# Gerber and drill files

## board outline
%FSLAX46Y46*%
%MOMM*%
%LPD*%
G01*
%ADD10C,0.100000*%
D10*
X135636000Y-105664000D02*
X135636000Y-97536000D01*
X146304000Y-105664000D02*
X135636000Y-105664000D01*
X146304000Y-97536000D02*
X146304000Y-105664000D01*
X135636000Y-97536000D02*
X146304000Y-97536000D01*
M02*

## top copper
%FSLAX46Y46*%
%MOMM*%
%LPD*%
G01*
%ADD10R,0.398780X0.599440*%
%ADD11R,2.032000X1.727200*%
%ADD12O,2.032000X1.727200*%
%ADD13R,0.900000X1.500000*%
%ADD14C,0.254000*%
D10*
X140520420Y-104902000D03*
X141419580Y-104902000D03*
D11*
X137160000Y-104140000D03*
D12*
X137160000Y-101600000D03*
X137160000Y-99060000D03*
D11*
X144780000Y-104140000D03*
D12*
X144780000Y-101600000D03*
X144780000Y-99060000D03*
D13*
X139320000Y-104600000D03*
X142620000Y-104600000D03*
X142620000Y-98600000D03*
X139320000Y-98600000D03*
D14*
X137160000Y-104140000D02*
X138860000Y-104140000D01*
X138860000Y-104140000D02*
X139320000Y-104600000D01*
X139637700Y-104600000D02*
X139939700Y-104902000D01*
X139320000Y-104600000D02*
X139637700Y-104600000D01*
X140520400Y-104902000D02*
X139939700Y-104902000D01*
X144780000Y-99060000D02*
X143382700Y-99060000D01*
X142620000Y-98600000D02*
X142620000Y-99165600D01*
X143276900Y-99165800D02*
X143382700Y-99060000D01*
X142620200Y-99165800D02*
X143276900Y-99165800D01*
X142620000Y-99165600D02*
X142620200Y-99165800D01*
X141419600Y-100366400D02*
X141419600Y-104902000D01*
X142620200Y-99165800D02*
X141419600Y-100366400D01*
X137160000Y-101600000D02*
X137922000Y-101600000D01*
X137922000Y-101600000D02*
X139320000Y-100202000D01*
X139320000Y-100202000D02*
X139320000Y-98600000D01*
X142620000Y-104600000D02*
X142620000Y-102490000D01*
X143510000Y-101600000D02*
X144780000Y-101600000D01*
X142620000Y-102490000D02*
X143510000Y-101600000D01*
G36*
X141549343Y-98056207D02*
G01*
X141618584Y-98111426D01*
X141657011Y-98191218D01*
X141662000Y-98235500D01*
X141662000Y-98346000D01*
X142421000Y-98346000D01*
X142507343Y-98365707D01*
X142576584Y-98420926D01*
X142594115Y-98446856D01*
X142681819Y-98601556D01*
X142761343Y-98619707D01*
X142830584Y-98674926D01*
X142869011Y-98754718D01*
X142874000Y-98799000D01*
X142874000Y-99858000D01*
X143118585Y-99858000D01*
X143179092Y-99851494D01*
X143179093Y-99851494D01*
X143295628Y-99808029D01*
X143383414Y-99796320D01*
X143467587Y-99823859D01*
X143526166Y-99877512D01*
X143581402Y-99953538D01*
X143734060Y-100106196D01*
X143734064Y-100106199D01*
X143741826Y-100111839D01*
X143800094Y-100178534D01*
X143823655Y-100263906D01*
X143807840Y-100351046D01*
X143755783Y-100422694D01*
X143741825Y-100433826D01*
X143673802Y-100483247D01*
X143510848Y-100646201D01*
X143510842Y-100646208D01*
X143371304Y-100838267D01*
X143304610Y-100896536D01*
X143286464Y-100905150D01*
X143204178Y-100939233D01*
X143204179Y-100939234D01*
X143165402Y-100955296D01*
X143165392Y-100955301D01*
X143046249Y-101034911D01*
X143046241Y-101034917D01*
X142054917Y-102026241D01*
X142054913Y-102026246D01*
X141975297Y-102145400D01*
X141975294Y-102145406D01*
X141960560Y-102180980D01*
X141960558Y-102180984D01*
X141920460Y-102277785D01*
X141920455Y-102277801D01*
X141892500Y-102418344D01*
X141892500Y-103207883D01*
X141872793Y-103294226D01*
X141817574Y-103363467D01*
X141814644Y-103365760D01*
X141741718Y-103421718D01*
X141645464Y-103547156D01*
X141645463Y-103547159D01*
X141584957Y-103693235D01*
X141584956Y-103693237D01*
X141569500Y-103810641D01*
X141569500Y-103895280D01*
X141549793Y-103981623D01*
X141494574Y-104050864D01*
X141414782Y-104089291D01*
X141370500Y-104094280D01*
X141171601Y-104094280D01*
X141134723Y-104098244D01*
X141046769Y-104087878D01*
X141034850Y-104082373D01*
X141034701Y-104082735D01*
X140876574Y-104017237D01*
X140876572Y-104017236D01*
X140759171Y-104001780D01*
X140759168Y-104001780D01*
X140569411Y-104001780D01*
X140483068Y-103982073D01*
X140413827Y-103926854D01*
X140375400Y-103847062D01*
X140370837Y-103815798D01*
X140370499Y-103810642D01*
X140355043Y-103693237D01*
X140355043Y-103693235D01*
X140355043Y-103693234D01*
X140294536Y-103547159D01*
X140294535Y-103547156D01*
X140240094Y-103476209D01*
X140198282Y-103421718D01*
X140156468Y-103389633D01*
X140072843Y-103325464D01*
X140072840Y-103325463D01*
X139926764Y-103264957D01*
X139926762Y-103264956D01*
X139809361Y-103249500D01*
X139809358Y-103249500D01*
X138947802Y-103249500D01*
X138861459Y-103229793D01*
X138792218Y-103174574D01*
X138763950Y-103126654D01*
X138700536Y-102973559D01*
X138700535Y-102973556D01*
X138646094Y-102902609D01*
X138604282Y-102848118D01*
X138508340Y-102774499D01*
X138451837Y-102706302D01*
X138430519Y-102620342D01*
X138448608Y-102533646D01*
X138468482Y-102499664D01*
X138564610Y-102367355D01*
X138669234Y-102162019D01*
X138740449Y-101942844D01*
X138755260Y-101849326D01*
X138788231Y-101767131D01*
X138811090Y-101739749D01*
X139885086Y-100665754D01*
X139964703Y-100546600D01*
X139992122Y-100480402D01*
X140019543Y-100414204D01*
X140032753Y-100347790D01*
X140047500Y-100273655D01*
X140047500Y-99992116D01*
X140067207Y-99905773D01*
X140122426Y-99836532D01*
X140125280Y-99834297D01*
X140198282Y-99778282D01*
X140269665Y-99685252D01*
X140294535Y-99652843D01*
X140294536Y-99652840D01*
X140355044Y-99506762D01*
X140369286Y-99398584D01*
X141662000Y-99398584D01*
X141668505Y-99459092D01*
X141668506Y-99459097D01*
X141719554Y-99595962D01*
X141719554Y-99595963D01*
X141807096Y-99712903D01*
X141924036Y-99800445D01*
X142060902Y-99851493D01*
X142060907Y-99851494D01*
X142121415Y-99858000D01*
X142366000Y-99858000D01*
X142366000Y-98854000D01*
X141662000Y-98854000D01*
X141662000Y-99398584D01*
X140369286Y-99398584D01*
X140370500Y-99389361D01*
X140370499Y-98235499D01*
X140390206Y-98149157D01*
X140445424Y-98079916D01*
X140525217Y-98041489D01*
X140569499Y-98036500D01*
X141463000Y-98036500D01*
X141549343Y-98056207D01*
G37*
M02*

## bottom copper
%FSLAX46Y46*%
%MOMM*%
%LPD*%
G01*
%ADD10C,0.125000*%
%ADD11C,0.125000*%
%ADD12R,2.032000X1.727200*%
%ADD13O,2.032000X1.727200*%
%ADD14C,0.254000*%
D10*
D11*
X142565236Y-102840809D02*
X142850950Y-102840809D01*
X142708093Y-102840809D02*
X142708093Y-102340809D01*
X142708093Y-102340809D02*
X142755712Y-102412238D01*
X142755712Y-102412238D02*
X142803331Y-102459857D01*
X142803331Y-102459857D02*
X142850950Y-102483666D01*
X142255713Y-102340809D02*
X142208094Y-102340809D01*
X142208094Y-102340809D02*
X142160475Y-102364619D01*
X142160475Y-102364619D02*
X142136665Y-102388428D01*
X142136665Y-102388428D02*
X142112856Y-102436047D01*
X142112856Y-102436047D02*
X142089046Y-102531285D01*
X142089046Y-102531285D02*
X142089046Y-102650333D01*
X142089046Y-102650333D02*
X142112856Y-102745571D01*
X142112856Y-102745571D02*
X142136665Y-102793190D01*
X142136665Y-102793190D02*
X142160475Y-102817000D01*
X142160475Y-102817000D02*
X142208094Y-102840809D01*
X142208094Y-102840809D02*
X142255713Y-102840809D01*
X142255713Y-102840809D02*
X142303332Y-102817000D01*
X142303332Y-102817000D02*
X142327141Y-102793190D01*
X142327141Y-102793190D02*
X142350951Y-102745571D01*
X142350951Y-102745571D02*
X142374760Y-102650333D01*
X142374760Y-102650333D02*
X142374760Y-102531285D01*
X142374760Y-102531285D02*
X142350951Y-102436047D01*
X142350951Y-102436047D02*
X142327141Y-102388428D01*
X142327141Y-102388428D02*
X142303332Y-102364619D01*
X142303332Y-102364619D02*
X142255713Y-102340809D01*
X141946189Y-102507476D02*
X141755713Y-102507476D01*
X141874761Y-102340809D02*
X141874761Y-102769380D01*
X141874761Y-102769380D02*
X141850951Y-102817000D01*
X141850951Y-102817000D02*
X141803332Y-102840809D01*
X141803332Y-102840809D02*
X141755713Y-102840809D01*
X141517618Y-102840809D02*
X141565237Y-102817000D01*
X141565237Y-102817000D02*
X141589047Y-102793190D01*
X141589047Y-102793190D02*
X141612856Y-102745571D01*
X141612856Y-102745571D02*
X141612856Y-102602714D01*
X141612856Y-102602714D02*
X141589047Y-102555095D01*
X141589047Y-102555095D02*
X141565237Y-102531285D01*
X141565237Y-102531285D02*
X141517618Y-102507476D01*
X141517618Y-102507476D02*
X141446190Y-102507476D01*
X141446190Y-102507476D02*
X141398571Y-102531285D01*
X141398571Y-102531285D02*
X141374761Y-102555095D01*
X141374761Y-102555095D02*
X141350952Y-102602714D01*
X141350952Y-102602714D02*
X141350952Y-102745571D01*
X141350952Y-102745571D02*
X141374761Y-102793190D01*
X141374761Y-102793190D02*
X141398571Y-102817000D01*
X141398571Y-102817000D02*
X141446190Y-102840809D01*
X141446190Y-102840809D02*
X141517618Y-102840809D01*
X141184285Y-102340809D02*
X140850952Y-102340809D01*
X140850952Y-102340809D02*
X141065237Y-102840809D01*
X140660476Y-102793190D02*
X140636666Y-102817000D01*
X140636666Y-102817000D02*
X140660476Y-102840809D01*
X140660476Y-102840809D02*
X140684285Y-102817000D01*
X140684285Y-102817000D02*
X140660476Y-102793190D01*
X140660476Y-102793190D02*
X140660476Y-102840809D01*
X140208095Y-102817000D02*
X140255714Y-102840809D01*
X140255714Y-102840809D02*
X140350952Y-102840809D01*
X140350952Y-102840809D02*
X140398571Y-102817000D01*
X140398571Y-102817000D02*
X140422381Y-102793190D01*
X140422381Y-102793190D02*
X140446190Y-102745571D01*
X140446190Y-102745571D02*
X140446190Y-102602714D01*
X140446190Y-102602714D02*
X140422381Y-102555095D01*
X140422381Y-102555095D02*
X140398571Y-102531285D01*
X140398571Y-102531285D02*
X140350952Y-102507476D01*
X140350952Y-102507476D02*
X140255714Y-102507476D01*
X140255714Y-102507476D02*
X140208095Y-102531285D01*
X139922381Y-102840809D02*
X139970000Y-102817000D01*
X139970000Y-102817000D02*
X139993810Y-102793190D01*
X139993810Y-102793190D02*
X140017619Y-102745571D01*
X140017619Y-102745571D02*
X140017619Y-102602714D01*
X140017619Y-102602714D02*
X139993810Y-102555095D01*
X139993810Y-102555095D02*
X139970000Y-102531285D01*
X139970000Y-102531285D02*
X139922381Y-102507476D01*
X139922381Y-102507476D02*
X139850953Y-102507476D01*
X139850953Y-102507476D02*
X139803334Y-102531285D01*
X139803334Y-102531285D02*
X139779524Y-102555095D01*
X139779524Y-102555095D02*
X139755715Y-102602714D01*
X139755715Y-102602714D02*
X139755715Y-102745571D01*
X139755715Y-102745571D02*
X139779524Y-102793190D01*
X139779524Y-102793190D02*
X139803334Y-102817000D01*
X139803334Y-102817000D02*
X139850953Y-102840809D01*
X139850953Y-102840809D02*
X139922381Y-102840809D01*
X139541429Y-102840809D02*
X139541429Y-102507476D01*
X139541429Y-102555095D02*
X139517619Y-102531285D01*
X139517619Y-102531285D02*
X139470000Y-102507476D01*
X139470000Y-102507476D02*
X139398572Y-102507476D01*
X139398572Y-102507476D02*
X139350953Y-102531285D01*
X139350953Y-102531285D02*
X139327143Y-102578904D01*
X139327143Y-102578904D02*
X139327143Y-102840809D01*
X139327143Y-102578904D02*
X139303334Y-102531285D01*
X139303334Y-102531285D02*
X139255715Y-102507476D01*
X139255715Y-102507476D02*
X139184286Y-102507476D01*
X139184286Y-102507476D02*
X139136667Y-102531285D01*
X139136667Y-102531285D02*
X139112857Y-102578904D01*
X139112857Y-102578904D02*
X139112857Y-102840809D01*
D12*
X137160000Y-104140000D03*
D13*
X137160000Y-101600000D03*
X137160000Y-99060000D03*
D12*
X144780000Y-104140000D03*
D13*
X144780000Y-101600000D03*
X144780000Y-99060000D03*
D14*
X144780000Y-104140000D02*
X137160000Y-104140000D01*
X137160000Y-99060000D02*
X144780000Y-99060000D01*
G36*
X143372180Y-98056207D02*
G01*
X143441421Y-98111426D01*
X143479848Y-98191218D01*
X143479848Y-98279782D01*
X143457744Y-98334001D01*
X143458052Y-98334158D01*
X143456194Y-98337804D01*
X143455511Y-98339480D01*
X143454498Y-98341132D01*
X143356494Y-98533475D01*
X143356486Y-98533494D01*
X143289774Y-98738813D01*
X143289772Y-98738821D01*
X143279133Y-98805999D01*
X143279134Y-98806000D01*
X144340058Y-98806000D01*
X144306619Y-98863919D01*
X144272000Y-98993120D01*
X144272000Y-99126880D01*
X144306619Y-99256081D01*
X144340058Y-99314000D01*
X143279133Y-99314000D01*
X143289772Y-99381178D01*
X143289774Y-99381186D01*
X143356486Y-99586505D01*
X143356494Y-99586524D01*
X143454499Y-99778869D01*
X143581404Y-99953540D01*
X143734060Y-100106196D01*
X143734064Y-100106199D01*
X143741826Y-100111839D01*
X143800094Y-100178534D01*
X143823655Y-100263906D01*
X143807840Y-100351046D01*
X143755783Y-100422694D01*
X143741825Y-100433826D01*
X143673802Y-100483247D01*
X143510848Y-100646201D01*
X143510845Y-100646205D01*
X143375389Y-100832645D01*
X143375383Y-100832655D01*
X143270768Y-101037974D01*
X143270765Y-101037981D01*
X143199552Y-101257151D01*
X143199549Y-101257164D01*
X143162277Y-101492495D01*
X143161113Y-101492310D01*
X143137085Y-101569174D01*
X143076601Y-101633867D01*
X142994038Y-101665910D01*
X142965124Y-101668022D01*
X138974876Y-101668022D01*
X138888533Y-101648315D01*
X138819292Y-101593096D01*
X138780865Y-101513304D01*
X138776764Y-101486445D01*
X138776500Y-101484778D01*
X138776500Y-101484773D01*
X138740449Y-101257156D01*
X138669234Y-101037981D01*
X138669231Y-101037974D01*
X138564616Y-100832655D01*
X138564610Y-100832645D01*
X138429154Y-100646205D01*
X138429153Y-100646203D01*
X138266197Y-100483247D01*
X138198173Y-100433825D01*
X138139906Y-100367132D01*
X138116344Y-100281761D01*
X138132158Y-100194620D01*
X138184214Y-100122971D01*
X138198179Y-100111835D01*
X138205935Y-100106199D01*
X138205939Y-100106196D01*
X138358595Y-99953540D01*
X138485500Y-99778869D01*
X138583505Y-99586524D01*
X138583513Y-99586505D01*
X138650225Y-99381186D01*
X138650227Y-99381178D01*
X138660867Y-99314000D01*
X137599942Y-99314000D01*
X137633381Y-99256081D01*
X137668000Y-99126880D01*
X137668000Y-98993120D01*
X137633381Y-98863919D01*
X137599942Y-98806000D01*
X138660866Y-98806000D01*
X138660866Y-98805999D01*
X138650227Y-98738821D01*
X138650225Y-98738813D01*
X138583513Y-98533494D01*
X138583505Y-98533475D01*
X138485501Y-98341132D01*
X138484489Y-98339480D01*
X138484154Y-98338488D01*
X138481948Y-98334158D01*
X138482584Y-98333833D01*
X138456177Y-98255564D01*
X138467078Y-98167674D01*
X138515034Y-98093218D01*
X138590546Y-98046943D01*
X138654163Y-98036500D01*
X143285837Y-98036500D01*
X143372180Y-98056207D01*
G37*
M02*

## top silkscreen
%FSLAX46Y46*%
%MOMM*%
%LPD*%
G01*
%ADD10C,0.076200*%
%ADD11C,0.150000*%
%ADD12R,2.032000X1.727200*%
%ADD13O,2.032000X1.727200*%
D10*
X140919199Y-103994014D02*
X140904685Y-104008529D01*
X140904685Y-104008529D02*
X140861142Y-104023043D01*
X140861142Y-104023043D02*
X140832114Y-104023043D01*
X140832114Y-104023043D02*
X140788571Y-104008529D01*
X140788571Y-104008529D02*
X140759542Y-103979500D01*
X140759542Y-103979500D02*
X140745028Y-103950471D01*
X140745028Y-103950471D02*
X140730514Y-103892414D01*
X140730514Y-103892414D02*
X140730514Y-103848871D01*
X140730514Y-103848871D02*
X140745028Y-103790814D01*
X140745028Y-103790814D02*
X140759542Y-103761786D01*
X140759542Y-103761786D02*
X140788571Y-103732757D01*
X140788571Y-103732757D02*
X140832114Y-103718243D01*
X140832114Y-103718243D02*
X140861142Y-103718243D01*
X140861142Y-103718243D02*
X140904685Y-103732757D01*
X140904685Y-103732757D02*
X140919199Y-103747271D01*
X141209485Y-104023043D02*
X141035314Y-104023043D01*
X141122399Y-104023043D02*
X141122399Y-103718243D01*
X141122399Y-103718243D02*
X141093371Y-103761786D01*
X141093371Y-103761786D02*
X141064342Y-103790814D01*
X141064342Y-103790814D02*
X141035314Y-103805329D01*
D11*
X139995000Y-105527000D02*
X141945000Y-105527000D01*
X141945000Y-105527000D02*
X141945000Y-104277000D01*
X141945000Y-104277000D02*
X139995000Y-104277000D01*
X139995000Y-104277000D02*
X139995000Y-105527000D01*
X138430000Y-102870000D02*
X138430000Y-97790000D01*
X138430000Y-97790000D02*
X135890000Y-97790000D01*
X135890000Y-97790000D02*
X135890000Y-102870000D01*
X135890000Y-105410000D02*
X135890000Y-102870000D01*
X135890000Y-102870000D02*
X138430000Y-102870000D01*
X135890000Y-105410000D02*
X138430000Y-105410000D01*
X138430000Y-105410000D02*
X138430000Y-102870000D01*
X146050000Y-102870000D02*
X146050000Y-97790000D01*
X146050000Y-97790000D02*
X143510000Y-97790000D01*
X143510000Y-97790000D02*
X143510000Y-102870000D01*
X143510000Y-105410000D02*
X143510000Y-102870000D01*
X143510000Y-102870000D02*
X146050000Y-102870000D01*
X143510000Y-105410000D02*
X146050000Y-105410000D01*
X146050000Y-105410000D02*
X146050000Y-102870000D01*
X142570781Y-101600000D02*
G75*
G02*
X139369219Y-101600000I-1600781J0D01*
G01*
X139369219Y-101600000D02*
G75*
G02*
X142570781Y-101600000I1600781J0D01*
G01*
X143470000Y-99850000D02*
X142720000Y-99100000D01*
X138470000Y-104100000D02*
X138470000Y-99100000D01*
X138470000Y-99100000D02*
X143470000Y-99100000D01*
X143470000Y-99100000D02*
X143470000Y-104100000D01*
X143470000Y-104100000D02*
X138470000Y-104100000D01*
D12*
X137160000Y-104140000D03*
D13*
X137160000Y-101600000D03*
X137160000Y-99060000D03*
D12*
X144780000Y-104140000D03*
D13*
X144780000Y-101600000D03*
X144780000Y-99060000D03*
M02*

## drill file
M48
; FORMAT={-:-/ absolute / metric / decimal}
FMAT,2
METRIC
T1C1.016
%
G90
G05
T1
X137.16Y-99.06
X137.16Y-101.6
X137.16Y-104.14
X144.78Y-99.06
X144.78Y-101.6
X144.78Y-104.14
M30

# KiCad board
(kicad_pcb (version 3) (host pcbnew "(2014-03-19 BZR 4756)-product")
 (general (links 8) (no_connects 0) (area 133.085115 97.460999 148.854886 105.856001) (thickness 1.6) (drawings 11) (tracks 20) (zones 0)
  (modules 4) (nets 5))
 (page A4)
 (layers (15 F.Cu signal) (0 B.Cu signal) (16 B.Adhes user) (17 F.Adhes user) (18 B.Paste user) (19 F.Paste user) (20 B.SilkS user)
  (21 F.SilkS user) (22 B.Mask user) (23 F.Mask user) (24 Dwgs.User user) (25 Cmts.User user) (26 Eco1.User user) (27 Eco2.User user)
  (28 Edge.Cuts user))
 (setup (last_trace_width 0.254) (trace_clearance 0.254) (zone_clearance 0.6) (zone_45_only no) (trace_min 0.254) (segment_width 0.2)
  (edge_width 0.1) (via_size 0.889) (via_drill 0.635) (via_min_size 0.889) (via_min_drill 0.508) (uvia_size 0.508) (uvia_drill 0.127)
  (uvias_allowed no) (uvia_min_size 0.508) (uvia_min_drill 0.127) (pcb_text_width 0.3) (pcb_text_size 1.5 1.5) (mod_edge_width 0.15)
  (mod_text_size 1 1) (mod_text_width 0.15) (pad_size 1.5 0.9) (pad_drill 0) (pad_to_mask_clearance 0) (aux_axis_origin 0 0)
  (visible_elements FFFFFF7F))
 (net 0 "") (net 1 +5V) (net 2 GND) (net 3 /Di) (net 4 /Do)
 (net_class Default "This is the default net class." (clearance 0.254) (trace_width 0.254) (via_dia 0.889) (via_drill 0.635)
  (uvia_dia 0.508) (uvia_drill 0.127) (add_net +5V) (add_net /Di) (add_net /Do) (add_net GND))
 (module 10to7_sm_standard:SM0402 (layer F.Cu) (at 140.97 104.902)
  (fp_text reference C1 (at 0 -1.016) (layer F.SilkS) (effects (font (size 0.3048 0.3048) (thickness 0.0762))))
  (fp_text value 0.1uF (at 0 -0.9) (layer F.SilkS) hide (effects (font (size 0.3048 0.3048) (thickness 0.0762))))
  (fp_line (start -0.975 0.625) (end 0.975 0.625) (layer F.SilkS) (width 0.15))
  (fp_line (start 0.975 0.625) (end 0.975 -0.625) (layer F.SilkS) (width 0.15))
  (fp_line (start 0.975 -0.625) (end -0.975 -0.625) (layer F.SilkS) (width 0.15))
  (fp_line (start -0.975 -0.625) (end -0.975 0.625) (layer F.SilkS) (width 0.15))
  (pad 1 smd rect (at -0.44958 0) (size 0.39878 0.59944) (layers F.Cu F.Paste F.Mask) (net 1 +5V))
  (pad 2 smd rect (at 0.44958 0) (size 0.39878 0.59944) (layers F.Cu F.Paste F.Mask) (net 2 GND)))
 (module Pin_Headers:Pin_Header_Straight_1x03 (layer F.Cu) (at 137.16 101.6 90)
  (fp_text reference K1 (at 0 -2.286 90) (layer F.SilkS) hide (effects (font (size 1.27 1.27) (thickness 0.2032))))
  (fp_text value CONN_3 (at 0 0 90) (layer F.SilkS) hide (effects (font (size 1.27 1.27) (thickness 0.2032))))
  (fp_line (start -1.27 1.27) (end 3.81 1.27) (layer F.SilkS) (width 0.15))
  (fp_line (start 3.81 1.27) (end 3.81 -1.27) (layer F.SilkS) (width 0.15))
  (fp_line (start 3.81 -1.27) (end -1.27 -1.27) (layer F.SilkS) (width 0.15))
  (fp_line (start -3.81 -1.27) (end -1.27 -1.27) (layer F.SilkS) (width 0.15))
  (fp_line (start -1.27 -1.27) (end -1.27 1.27) (layer F.SilkS) (width 0.15))
  (fp_line (start -3.81 -1.27) (end -3.81 1.27) (layer F.SilkS) (width 0.15))
  (fp_line (start -3.81 1.27) (end -1.27 1.27) (layer F.SilkS) (width 0.15))
  (pad 1 thru_hole rect (at -2.54 0 90) (size 1.7272 2.032) (drill 1.016) (layers *.Cu *.Mask F.SilkS) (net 1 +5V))
  (pad 2 thru_hole oval (at 0 0 90) (size 1.7272 2.032) (drill 1.016) (layers *.Cu *.Mask F.SilkS) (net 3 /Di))
  (pad 3 thru_hole oval (at 2.54 0 90) (size 1.7272 2.032) (drill 1.016) (layers *.Cu *.Mask F.SilkS) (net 2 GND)))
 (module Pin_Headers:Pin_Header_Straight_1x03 (layer F.Cu) (at 144.78 101.6 90)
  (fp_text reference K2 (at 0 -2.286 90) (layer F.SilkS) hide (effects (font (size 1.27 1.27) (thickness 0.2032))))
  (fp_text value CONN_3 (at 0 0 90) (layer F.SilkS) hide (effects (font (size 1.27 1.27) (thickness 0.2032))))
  (fp_line (start -1.27 1.27) (end 3.81 1.27) (layer F.SilkS) (width 0.15))
  (fp_line (start 3.81 1.27) (end 3.81 -1.27) (layer F.SilkS) (width 0.15))
  (fp_line (start 3.81 -1.27) (end -1.27 -1.27) (layer F.SilkS) (width 0.15))
  (fp_line (start -3.81 -1.27) (end -1.27 -1.27) (layer F.SilkS) (width 0.15))
  (fp_line (start -1.27 -1.27) (end -1.27 1.27) (layer F.SilkS) (width 0.15))
  (fp_line (start -3.81 -1.27) (end -3.81 1.27) (layer F.SilkS) (width 0.15))
  (fp_line (start -3.81 1.27) (end -1.27 1.27) (layer F.SilkS) (width 0.15))
  (pad 1 thru_hole rect (at -2.54 0 90) (size 1.7272 2.032) (drill 1.016) (layers *.Cu *.Mask F.SilkS) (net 1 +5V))
  (pad 2 thru_hole oval (at 0 0 90) (size 1.7272 2.032) (drill 1.016) (layers *.Cu *.Mask F.SilkS) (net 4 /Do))
  (pad 3 thru_hole oval (at 2.54 0 90) (size 1.7272 2.032) (drill 1.016) (layers *.Cu *.Mask F.SilkS) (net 2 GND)))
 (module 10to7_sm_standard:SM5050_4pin (layer F.Cu) (at 140.97 101.6 90)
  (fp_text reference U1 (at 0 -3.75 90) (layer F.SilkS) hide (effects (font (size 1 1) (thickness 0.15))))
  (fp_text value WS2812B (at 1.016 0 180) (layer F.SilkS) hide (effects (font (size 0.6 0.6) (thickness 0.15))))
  (fp_circle (center 0 0) (end 1 -1.25) (layer F.SilkS) (width 0.15))
  (fp_line (start 1.75 2.5) (end 2.5 1.75) (layer F.SilkS) (width 0.15))
  (fp_line (start -2.5 -2.5) (end 2.5 -2.5) (layer F.SilkS) (width 0.15))
  (fp_line (start 2.5 -2.5) (end 2.5 2.5) (layer F.SilkS) (width 0.15))
  (fp_line (start 2.5 2.5) (end -2.5 2.5) (layer F.SilkS) (width 0.15))
  (fp_line (start -2.5 2.5) (end -2.5 -2.5) (layer F.SilkS) (width 0.15))
  (pad 1 smd rect (at -3 -1.65 90) (size 1.5 0.9) (layers F.Cu F.Paste F.Mask) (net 1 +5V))
  (pad 2 smd rect (at -3 1.65 90) (size 1.5 0.9) (layers F.Cu F.Paste F.Mask) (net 4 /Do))
  (pad 3 smd rect (at 3 1.65 90) (size 1.5 0.9) (layers F.Cu F.Paste F.Mask) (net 2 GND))
  (pad 4 smd rect (at 3 -1.65 90) (size 1.5 0.9) (layers F.Cu F.Paste F.Mask) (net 3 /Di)))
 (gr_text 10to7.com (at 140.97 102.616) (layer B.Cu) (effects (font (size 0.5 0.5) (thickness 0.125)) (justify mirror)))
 (gr_line (start 135.636 105.664) (end 135.636 97.536) (angle 90) (layer Edge.Cuts) (width 0.1))
 (gr_line (start 146.304 105.664) (end 135.636 105.664) (angle 90) (layer Edge.Cuts) (width 0.1))
 (gr_line (start 146.304 97.536) (end 146.304 105.664) (angle 90) (layer Edge.Cuts) (width 0.1))
 (gr_line (start 135.636 97.536) (end 146.304 97.536) (angle 90) (layer Edge.Cuts) (width 0.1))
 (segment (start 137.16 104.14) (end 138.86 104.14) (width 0.254) (layer F.Cu) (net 1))
 (segment (start 138.86 104.14) (end 139.32 104.6) (width 0.254) (layer F.Cu) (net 1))
 (segment (start 139.6377 104.6) (end 139.9397 104.902) (width 0.254) (layer F.Cu) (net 1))
 (segment (start 139.32 104.6) (end 139.6377 104.6) (width 0.254) (layer F.Cu) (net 1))
 (segment (start 140.5204 104.902) (end 139.9397 104.902) (width 0.254) (layer F.Cu) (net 1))
 (segment (start 144.78 104.14) (end 137.16 104.14) (width 0.254) (layer B.Cu) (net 1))
 (segment (start 144.78 99.06) (end 143.3827 99.06) (width 0.254) (layer F.Cu) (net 2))
 (segment (start 142.62 98.6) (end 142.62 99.1656) (width 0.254) (layer F.Cu) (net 2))
 (segment (start 143.2769 99.1658) (end 143.3827 99.06) (width 0.254) (layer F.Cu) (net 2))
 (segment (start 142.6202 99.1658) (end 143.2769 99.1658) (width 0.254) (layer F.Cu) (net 2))
 (segment (start 142.62 99.1656) (end 142.6202 99.1658) (width 0.254) (layer F.Cu) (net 2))
 (segment (start 141.4196 100.3664) (end 141.4196 104.902) (width 0.254) (layer F.Cu) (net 2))
 (segment (start 142.6202 99.1658) (end 141.4196 100.3664) (width 0.254) (layer F.Cu) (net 2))
 (segment (start 137.16 99.06) (end 144.78 99.06) (width 0.254) (layer B.Cu) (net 2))
 (segment (start 137.16 101.6) (end 137.922 101.6) (width 0.254) (layer F.Cu) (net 3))
 (segment (start 137.922 101.6) (end 139.32 100.202) (width 0.254) (layer F.Cu) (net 3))
 (segment (start 139.32 100.202) (end 139.32 98.6) (width 0.254) (layer F.Cu) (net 3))
 (segment (start 142.62 104.6) (end 142.62 102.49) (width 0.254) (layer F.Cu) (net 4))
 (segment (start 143.51 101.6) (end 144.78 101.6) (width 0.254) (layer F.Cu) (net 4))
 (segment (start 142.62 102.49) (end 143.51 101.6) (width 0.254) (layer F.Cu) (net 4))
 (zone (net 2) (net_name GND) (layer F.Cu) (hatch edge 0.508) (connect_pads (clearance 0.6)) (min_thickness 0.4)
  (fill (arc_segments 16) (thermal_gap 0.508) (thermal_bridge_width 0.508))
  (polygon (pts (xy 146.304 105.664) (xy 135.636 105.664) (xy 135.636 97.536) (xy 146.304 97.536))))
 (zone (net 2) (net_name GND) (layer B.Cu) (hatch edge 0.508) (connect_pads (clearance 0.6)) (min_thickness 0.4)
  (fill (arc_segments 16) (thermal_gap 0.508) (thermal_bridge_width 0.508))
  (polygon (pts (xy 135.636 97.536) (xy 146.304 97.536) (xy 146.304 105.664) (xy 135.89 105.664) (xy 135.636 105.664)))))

